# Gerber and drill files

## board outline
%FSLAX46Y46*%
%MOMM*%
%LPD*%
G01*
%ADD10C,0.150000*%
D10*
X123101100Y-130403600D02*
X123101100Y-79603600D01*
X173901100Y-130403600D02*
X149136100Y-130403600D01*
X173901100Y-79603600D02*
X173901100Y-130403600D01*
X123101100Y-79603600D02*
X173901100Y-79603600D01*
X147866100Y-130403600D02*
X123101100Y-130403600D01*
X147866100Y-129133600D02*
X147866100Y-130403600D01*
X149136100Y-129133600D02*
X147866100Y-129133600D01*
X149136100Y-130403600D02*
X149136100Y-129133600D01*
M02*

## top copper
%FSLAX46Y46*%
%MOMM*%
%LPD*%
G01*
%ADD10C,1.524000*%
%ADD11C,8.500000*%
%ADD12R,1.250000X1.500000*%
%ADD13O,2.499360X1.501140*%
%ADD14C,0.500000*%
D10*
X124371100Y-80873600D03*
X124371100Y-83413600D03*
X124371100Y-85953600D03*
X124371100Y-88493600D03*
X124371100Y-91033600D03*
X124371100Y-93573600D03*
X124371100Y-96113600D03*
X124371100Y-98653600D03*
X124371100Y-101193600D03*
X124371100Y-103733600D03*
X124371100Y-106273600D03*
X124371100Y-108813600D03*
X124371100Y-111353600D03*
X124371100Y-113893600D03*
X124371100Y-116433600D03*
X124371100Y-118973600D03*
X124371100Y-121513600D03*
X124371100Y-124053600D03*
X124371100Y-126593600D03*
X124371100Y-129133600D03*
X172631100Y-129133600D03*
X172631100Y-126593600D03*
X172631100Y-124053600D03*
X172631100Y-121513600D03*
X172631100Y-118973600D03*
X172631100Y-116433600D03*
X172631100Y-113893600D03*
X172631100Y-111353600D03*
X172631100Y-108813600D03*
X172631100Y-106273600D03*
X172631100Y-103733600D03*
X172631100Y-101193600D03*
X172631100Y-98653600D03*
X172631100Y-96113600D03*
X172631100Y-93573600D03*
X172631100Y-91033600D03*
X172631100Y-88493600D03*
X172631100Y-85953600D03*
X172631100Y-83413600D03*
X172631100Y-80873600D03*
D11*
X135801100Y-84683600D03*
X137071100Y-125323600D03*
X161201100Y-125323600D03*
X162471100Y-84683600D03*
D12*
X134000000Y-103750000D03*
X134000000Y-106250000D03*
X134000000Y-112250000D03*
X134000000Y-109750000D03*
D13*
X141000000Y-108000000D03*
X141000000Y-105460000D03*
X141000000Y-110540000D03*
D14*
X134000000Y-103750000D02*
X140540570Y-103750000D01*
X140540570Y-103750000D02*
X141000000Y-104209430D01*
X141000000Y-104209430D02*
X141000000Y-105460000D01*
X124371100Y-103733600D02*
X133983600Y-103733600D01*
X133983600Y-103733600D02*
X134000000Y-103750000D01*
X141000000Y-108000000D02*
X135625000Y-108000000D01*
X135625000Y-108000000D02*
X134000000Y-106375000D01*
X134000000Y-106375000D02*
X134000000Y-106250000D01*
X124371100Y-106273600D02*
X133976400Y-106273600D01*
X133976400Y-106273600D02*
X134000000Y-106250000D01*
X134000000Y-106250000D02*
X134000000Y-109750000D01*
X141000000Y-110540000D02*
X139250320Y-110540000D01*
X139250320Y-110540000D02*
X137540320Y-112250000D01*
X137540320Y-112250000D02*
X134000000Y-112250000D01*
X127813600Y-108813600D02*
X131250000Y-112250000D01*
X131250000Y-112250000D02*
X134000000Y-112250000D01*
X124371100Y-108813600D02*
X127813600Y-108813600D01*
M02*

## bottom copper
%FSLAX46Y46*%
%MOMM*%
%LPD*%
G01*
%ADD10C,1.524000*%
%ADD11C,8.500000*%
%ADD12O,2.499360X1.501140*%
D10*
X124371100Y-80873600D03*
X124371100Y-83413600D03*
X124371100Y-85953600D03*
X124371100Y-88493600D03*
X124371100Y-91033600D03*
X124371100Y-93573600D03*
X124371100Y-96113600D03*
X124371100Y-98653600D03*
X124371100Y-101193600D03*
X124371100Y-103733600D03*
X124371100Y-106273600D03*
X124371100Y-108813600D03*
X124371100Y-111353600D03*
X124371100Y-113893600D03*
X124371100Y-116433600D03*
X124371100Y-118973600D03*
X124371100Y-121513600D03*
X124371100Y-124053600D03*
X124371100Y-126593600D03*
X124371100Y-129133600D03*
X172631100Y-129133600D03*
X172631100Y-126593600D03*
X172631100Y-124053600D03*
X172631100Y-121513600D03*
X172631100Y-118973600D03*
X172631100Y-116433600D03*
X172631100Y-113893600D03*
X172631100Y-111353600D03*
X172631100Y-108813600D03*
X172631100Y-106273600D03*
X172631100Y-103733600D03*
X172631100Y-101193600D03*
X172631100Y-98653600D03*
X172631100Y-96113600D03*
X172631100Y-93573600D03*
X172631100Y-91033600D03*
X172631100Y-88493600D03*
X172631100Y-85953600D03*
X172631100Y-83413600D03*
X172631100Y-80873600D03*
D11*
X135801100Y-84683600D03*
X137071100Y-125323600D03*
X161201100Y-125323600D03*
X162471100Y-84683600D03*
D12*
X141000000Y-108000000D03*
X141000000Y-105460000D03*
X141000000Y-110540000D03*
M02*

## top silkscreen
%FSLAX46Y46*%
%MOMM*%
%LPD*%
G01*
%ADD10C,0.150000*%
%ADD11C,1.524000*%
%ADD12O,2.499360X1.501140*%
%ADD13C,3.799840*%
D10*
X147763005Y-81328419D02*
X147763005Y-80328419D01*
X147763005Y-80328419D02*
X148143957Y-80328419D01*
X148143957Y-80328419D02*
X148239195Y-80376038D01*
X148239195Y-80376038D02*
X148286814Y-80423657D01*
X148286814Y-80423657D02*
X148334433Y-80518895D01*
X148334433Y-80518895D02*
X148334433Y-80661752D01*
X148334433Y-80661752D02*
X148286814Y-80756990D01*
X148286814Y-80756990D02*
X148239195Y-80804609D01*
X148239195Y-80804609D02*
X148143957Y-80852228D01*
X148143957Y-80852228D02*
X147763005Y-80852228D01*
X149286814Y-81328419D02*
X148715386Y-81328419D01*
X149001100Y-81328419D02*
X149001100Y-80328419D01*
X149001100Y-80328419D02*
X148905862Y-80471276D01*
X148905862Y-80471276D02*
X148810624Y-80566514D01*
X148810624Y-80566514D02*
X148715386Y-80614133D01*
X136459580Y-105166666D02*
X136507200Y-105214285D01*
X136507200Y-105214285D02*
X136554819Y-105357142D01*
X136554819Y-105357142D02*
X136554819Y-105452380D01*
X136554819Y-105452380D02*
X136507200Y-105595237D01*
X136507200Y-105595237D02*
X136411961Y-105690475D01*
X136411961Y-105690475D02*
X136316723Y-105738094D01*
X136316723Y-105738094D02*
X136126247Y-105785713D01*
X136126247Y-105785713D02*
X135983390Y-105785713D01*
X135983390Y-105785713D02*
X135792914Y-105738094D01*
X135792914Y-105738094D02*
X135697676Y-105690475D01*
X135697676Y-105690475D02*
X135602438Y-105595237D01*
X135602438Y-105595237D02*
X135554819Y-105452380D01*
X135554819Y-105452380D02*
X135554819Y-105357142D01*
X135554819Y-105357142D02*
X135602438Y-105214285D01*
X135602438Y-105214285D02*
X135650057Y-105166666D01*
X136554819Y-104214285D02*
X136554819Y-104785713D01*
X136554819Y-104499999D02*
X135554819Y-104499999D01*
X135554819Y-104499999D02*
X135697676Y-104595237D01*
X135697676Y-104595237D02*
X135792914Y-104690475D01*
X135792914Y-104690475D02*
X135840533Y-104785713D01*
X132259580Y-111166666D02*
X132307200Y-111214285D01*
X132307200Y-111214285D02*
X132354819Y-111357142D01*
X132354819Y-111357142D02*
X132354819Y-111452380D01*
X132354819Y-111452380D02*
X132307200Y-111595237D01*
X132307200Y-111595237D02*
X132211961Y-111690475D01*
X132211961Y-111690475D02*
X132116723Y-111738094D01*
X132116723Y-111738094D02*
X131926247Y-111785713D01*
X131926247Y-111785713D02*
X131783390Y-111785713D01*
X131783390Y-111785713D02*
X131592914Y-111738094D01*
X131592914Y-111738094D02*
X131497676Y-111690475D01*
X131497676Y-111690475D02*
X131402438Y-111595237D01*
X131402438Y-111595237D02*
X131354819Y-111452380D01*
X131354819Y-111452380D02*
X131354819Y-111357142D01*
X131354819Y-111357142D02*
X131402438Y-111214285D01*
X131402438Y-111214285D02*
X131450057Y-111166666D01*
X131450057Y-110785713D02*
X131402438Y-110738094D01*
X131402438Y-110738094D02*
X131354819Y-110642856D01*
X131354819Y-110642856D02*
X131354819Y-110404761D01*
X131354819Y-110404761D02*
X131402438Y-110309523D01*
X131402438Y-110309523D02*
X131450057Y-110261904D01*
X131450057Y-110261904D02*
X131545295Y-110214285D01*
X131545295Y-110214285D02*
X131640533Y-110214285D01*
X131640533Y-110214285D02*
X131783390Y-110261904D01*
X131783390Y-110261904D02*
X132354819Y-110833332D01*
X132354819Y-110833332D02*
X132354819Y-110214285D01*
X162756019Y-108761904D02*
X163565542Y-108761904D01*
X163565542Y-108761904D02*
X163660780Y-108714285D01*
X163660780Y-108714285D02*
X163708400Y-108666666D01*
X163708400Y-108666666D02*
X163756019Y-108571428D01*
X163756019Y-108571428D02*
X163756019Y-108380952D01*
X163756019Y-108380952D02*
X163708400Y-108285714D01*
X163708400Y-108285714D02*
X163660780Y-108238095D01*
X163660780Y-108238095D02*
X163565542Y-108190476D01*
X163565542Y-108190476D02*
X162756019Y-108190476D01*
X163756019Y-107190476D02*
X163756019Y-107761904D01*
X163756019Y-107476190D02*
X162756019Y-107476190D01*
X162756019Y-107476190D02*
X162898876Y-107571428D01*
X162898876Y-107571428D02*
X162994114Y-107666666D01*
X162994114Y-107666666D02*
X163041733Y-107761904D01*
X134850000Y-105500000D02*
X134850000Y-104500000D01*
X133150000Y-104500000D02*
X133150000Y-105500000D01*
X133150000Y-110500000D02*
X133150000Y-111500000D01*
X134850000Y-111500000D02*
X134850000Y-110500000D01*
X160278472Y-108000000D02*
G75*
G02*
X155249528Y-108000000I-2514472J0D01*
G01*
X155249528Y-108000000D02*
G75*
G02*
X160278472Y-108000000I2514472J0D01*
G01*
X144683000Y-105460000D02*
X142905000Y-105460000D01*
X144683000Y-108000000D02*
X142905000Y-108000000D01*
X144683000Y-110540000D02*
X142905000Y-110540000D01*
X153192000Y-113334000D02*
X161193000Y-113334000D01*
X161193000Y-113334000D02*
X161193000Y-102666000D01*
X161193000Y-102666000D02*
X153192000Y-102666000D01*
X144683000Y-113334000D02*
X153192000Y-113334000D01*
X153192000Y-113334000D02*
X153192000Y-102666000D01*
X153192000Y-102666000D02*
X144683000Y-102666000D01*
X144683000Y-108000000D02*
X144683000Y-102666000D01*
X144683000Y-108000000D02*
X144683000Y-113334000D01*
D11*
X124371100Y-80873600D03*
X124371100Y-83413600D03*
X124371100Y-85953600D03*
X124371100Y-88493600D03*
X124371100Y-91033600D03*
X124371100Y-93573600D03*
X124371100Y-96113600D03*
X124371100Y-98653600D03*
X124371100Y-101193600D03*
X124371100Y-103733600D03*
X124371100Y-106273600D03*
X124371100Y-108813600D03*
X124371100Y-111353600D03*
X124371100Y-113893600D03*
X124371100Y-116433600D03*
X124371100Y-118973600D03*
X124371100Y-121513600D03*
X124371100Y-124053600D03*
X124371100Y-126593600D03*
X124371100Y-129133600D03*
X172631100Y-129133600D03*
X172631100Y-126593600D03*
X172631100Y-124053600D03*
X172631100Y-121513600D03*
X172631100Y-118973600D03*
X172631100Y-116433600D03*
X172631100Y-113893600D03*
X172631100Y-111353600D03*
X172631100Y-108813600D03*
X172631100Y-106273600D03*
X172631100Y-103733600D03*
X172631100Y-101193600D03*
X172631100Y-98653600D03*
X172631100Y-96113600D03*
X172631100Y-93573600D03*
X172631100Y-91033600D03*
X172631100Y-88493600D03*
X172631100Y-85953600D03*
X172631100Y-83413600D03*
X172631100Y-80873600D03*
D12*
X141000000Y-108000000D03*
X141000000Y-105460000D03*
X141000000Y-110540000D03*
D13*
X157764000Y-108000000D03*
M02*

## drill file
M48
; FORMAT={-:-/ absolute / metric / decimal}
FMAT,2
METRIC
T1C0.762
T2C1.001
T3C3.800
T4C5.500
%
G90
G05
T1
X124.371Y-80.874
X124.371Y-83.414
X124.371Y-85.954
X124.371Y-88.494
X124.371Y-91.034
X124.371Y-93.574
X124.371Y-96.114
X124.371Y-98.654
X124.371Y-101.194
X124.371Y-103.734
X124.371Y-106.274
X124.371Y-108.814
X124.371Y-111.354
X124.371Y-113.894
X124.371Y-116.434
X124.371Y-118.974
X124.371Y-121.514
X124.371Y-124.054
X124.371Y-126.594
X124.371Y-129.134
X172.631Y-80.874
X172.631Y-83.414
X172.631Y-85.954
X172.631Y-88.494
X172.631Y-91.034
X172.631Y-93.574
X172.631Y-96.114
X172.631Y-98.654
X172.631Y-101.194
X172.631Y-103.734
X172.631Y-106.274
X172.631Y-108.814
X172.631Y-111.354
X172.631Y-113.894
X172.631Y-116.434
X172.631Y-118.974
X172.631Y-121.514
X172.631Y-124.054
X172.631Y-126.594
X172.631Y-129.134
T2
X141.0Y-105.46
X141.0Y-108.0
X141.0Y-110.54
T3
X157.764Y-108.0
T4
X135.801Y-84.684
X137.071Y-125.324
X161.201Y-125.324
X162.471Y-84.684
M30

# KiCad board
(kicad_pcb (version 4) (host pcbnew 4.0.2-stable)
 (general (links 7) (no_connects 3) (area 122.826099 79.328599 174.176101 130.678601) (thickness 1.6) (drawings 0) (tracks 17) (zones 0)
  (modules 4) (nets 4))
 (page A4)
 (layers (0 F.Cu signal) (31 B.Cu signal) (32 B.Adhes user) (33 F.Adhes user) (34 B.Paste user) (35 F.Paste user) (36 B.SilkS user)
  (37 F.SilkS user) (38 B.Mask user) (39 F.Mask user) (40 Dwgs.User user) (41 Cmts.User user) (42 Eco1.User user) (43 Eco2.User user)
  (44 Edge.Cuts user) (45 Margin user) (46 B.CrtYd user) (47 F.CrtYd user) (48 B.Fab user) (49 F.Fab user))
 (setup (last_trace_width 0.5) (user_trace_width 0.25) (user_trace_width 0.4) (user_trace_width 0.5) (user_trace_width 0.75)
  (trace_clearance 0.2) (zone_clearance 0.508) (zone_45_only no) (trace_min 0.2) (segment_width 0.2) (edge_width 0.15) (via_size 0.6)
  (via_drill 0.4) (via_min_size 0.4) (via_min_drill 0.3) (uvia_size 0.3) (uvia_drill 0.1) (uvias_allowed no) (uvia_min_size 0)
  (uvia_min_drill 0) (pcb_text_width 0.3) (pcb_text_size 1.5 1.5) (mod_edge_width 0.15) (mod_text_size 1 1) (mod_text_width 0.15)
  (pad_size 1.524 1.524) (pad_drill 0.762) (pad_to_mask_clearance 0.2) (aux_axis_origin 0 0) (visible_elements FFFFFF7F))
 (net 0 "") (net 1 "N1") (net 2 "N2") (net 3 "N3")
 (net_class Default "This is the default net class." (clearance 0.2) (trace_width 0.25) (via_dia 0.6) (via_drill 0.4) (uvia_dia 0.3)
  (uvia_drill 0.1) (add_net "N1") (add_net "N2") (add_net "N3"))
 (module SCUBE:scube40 (layer F.Cu) (at 148.5011 105.0036)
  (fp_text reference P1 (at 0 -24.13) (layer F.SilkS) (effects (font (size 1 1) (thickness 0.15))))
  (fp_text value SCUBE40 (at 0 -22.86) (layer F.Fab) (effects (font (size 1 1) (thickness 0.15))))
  (fp_line (start -25.4 25.4) (end -25.4 -25.4) (layer Edge.Cuts) (width 0.15))
  (fp_line (start 25.4 25.4) (end 0.635 25.4) (layer Edge.Cuts) (width 0.15))
  (fp_line (start 25.4 -25.4) (end 25.4 25.4) (layer Edge.Cuts) (width 0.15))
  (fp_line (start -25.4 -25.4) (end 25.4 -25.4) (layer Edge.Cuts) (width 0.15))
  (fp_line (start -0.635 25.4) (end -25.4 25.4) (layer Edge.Cuts) (width 0.15))
  (fp_line (start -0.635 24.13) (end -0.635 25.4) (layer Edge.Cuts) (width 0.15))
  (fp_line (start 0.635 24.13) (end -0.635 24.13) (layer Edge.Cuts) (width 0.15))
  (fp_line (start 0.635 25.4) (end 0.635 24.13) (layer Edge.Cuts) (width 0.15))
  (pad 1 thru_hole circle (at -24.13 -24.13) (size 1.524 1.524) (drill 0.762) (layers *.Cu *.Mask F.SilkS))
  (pad 2 thru_hole circle (at -24.13 -21.59) (size 1.524 1.524) (drill 0.762) (layers *.Cu *.Mask F.SilkS))
  (pad 3 thru_hole circle (at -24.13 -19.05) (size 1.524 1.524) (drill 0.762) (layers *.Cu *.Mask F.SilkS))
  (pad 4 thru_hole circle (at -24.13 -16.51) (size 1.524 1.524) (drill 0.762) (layers *.Cu *.Mask F.SilkS))
  (pad 5 thru_hole circle (at -24.13 -13.97) (size 1.524 1.524) (drill 0.762) (layers *.Cu *.Mask F.SilkS))
  (pad 6 thru_hole circle (at -24.13 -11.43) (size 1.524 1.524) (drill 0.762) (layers *.Cu *.Mask F.SilkS))
  (pad 7 thru_hole circle (at -24.13 -8.89) (size 1.524 1.524) (drill 0.762) (layers *.Cu *.Mask F.SilkS))
  (pad 8 thru_hole circle (at -24.13 -6.35) (size 1.524 1.524) (drill 0.762) (layers *.Cu *.Mask F.SilkS))
  (pad 9 thru_hole circle (at -24.13 -3.81) (size 1.524 1.524) (drill 0.762) (layers *.Cu *.Mask F.SilkS))
  (pad 10 thru_hole circle (at -24.13 -1.27) (size 1.524 1.524) (drill 0.762) (layers *.Cu *.Mask F.SilkS) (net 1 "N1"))
  (pad 11 thru_hole circle (at -24.13 1.27) (size 1.524 1.524) (drill 0.762) (layers *.Cu *.Mask F.SilkS) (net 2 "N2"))
  (pad 12 thru_hole circle (at -24.13 3.81) (size 1.524 1.524) (drill 0.762) (layers *.Cu *.Mask F.SilkS) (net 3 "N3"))
  (pad 13 thru_hole circle (at -24.13 6.35) (size 1.524 1.524) (drill 0.762) (layers *.Cu *.Mask F.SilkS))
  (pad 14 thru_hole circle (at -24.13 8.89) (size 1.524 1.524) (drill 0.762) (layers *.Cu *.Mask F.SilkS))
  (pad 15 thru_hole circle (at -24.13 11.43) (size 1.524 1.524) (drill 0.762) (layers *.Cu *.Mask F.SilkS))
  (pad 16 thru_hole circle (at -24.13 13.97) (size 1.524 1.524) (drill 0.762) (layers *.Cu *.Mask F.SilkS))
  (pad 17 thru_hole circle (at -24.13 16.51) (size 1.524 1.524) (drill 0.762) (layers *.Cu *.Mask F.SilkS))
  (pad 18 thru_hole circle (at -24.13 19.05) (size 1.524 1.524) (drill 0.762) (layers *.Cu *.Mask F.SilkS))
  (pad 19 thru_hole circle (at -24.13 21.59) (size 1.524 1.524) (drill 0.762) (layers *.Cu *.Mask F.SilkS))
  (pad 20 thru_hole circle (at -24.13 24.13) (size 1.524 1.524) (drill 0.762) (layers *.Cu *.Mask F.SilkS))
  (pad 21 thru_hole circle (at 24.13 24.13) (size 1.524 1.524) (drill 0.762) (layers *.Cu *.Mask F.SilkS))
  (pad 22 thru_hole circle (at 24.13 21.59) (size 1.524 1.524) (drill 0.762) (layers *.Cu *.Mask F.SilkS))
  (pad 23 thru_hole circle (at 24.13 19.05) (size 1.524 1.524) (drill 0.762) (layers *.Cu *.Mask F.SilkS))
  (pad 24 thru_hole circle (at 24.13 16.51) (size 1.524 1.524) (drill 0.762) (layers *.Cu *.Mask F.SilkS))
  (pad 25 thru_hole circle (at 24.13 13.97) (size 1.524 1.524) (drill 0.762) (layers *.Cu *.Mask F.SilkS))
  (pad 26 thru_hole circle (at 24.13 11.43) (size 1.524 1.524) (drill 0.762) (layers *.Cu *.Mask F.SilkS))
  (pad 27 thru_hole circle (at 24.13 8.89) (size 1.524 1.524) (drill 0.762) (layers *.Cu *.Mask F.SilkS))
  (pad 28 thru_hole circle (at 24.13 6.35) (size 1.524 1.524) (drill 0.762) (layers *.Cu *.Mask F.SilkS))
  (pad 29 thru_hole circle (at 24.13 3.81) (size 1.524 1.524) (drill 0.762) (layers *.Cu *.Mask F.SilkS))
  (pad 30 thru_hole circle (at 24.13 1.27) (size 1.524 1.524) (drill 0.762) (layers *.Cu *.Mask F.SilkS))
  (pad 31 thru_hole circle (at 24.13 -1.27) (size 1.524 1.524) (drill 0.762) (layers *.Cu *.Mask F.SilkS))
  (pad 32 thru_hole circle (at 24.13 -3.81) (size 1.524 1.524) (drill 0.762) (layers *.Cu *.Mask F.SilkS))
  (pad 33 thru_hole circle (at 24.13 -6.35) (size 1.524 1.524) (drill 0.762) (layers *.Cu *.Mask F.SilkS))
  (pad 34 thru_hole circle (at 24.13 -8.89) (size 1.524 1.524) (drill 0.762) (layers *.Cu *.Mask F.SilkS))
  (pad 35 thru_hole circle (at 24.13 -11.43) (size 1.524 1.524) (drill 0.762) (layers *.Cu *.Mask F.SilkS))
  (pad 36 thru_hole circle (at 24.13 -13.97) (size 1.524 1.524) (drill 0.762) (layers *.Cu *.Mask F.SilkS))
  (pad 37 thru_hole circle (at 24.13 -16.51) (size 1.524 1.524) (drill 0.762) (layers *.Cu *.Mask F.SilkS))
  (pad 38 thru_hole circle (at 24.13 -19.05) (size 1.524 1.524) (drill 0.762) (layers *.Cu *.Mask F.SilkS))
  (pad 39 thru_hole circle (at 24.13 -21.59) (size 1.524 1.524) (drill 0.762) (layers *.Cu *.Mask F.SilkS))
  (pad 40 thru_hole circle (at 24.13 -24.13) (size 1.524 1.524) (drill 0.762) (layers *.Cu *.Mask F.SilkS))
  (pad "" np_thru_hole circle (at -12.7 -20.32) (size 8.5 8.5) (drill 5.5) (layers *.Cu))
  (pad "" np_thru_hole circle (at -11.43 20.32) (size 8.5 8.5) (drill 5.5) (layers *.Cu))
  (pad "" np_thru_hole circle (at 12.7 20.32) (size 8.5 8.5) (drill 5.5) (layers *.Cu))
  (pad "" np_thru_hole circle (at 13.97 -20.32) (size 8.5 8.5) (drill 5.5) (layers *.Cu)))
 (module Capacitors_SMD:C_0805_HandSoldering (layer F.Cu) (at 134 105 270)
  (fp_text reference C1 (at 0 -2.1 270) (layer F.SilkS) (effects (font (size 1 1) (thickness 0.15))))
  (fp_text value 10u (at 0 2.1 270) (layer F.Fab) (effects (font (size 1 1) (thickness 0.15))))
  (fp_line (start 0.5 -0.85) (end -0.5 -0.85) (layer F.SilkS) (width 0.15))
  (fp_line (start -0.5 0.85) (end 0.5 0.85) (layer F.SilkS) (width 0.15))
  (pad 1 smd rect (at -1.25 0 270) (size 1.5 1.25) (layers F.Cu F.Paste F.Mask) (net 1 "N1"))
  (pad 2 smd rect (at 1.25 0 270) (size 1.5 1.25) (layers F.Cu F.Paste F.Mask) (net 2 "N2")))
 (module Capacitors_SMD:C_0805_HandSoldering (layer F.Cu) (at 134 111 90)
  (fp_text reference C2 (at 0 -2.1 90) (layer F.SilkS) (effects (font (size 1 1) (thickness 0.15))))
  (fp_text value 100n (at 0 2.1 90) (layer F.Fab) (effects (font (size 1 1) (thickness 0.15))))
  (fp_line (start 0.5 -0.85) (end -0.5 -0.85) (layer F.SilkS) (width 0.15))
  (fp_line (start -0.5 0.85) (end 0.5 0.85) (layer F.SilkS) (width 0.15))
  (pad 1 smd rect (at -1.25 0 90) (size 1.5 1.25) (layers F.Cu F.Paste F.Mask) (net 3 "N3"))
  (pad 2 smd rect (at 1.25 0 90) (size 1.5 1.25) (layers F.Cu F.Paste F.Mask) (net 2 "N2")))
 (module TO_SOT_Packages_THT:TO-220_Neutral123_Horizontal (layer F.Cu) (at 141 108 270)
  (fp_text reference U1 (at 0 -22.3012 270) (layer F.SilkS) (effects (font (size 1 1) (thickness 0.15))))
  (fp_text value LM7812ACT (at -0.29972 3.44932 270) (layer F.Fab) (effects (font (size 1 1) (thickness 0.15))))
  (fp_circle (center 0 -16.764) (end 1.778 -14.986) (layer F.SilkS) (width 0.15))
  (fp_line (start -2.54 -3.683) (end -2.54 -1.905) (layer F.SilkS) (width 0.15))
  (fp_line (start 0 -3.683) (end 0 -1.905) (layer F.SilkS) (width 0.15))
  (fp_line (start 2.54 -3.683) (end 2.54 -1.905) (layer F.SilkS) (width 0.15))
  (fp_line (start 5.334 -12.192) (end 5.334 -20.193) (layer F.SilkS) (width 0.15))
  (fp_line (start 5.334 -20.193) (end -5.334 -20.193) (layer F.SilkS) (width 0.15))
  (fp_line (start -5.334 -20.193) (end -5.334 -12.192) (layer F.SilkS) (width 0.15))
  (fp_line (start 5.334 -3.683) (end 5.334 -12.192) (layer F.SilkS) (width 0.15))
  (fp_line (start 5.334 -12.192) (end -5.334 -12.192) (layer F.SilkS) (width 0.15))
  (fp_line (start -5.334 -12.192) (end -5.334 -3.683) (layer F.SilkS) (width 0.15))
  (fp_line (start 0 -3.683) (end -5.334 -3.683) (layer F.SilkS) (width 0.15))
  (fp_line (start 0 -3.683) (end 5.334 -3.683) (layer F.SilkS) (width 0.15))
  (pad 2 thru_hole oval (at 0 0) (size 2.49936 1.50114) (drill 1.00076) (layers *.Cu *.Mask F.SilkS) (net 2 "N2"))
  (pad 1 thru_hole oval (at -2.54 0) (size 2.49936 1.50114) (drill 1.00076) (layers *.Cu *.Mask F.SilkS) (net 1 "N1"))
  (pad 3 thru_hole oval (at 2.54 0) (size 2.49936 1.50114) (drill 1.00076) (layers *.Cu *.Mask F.SilkS) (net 3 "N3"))
  (pad "" np_thru_hole circle (at 0 -16.764) (size 3.79984 3.79984) (drill 3.79984) (layers *.Cu *.Mask F.SilkS)))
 (segment (start 134 103.75) (end 140.54057 103.75) (width 0.5) (layer F.Cu) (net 1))
 (segment (start 140.54057 103.75) (end 141 104.20943) (width 0.5) (layer F.Cu) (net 1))
 (segment (start 141 104.20943) (end 141 105.46) (width 0.5) (layer F.Cu) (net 1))
 (segment (start 124.3711 103.7336) (end 133.9836 103.7336) (width 0.5) (layer F.Cu) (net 1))
 (segment (start 133.9836 103.7336) (end 134 103.75) (width 0.5) (layer F.Cu) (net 1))
 (segment (start 141 108) (end 135.625 108) (width 0.5) (layer F.Cu) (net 2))
 (segment (start 135.625 108) (end 134 106.375) (width 0.5) (layer F.Cu) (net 2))
 (segment (start 134 106.375) (end 134 106.25) (width 0.5) (layer F.Cu) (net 2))
 (segment (start 124.3711 106.2736) (end 133.9764 106.2736) (width 0.5) (layer F.Cu) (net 2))
 (segment (start 133.9764 106.2736) (end 134 106.25) (width 0.5) (layer F.Cu) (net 2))
 (segment (start 134 106.25) (end 134 109.75) (width 0.5) (layer F.Cu) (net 2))
 (segment (start 141 110.54) (end 139.25032 110.54) (width 0.5) (layer F.Cu) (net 3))
 (segment (start 139.25032 110.54) (end 137.54032 112.25) (width 0.5) (layer F.Cu) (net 3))
 (segment (start 137.54032 112.25) (end 134 112.25) (width 0.5) (layer F.Cu) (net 3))
 (segment (start 127.8136 108.8136) (end 131.25 112.25) (width 0.5) (layer F.Cu) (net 3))
 (segment (start 131.25 112.25) (end 134 112.25) (width 0.5) (layer F.Cu) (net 3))
 (segment (start 124.3711 108.8136) (end 127.8136 108.8136) (width 0.5) (layer F.Cu) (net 3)))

